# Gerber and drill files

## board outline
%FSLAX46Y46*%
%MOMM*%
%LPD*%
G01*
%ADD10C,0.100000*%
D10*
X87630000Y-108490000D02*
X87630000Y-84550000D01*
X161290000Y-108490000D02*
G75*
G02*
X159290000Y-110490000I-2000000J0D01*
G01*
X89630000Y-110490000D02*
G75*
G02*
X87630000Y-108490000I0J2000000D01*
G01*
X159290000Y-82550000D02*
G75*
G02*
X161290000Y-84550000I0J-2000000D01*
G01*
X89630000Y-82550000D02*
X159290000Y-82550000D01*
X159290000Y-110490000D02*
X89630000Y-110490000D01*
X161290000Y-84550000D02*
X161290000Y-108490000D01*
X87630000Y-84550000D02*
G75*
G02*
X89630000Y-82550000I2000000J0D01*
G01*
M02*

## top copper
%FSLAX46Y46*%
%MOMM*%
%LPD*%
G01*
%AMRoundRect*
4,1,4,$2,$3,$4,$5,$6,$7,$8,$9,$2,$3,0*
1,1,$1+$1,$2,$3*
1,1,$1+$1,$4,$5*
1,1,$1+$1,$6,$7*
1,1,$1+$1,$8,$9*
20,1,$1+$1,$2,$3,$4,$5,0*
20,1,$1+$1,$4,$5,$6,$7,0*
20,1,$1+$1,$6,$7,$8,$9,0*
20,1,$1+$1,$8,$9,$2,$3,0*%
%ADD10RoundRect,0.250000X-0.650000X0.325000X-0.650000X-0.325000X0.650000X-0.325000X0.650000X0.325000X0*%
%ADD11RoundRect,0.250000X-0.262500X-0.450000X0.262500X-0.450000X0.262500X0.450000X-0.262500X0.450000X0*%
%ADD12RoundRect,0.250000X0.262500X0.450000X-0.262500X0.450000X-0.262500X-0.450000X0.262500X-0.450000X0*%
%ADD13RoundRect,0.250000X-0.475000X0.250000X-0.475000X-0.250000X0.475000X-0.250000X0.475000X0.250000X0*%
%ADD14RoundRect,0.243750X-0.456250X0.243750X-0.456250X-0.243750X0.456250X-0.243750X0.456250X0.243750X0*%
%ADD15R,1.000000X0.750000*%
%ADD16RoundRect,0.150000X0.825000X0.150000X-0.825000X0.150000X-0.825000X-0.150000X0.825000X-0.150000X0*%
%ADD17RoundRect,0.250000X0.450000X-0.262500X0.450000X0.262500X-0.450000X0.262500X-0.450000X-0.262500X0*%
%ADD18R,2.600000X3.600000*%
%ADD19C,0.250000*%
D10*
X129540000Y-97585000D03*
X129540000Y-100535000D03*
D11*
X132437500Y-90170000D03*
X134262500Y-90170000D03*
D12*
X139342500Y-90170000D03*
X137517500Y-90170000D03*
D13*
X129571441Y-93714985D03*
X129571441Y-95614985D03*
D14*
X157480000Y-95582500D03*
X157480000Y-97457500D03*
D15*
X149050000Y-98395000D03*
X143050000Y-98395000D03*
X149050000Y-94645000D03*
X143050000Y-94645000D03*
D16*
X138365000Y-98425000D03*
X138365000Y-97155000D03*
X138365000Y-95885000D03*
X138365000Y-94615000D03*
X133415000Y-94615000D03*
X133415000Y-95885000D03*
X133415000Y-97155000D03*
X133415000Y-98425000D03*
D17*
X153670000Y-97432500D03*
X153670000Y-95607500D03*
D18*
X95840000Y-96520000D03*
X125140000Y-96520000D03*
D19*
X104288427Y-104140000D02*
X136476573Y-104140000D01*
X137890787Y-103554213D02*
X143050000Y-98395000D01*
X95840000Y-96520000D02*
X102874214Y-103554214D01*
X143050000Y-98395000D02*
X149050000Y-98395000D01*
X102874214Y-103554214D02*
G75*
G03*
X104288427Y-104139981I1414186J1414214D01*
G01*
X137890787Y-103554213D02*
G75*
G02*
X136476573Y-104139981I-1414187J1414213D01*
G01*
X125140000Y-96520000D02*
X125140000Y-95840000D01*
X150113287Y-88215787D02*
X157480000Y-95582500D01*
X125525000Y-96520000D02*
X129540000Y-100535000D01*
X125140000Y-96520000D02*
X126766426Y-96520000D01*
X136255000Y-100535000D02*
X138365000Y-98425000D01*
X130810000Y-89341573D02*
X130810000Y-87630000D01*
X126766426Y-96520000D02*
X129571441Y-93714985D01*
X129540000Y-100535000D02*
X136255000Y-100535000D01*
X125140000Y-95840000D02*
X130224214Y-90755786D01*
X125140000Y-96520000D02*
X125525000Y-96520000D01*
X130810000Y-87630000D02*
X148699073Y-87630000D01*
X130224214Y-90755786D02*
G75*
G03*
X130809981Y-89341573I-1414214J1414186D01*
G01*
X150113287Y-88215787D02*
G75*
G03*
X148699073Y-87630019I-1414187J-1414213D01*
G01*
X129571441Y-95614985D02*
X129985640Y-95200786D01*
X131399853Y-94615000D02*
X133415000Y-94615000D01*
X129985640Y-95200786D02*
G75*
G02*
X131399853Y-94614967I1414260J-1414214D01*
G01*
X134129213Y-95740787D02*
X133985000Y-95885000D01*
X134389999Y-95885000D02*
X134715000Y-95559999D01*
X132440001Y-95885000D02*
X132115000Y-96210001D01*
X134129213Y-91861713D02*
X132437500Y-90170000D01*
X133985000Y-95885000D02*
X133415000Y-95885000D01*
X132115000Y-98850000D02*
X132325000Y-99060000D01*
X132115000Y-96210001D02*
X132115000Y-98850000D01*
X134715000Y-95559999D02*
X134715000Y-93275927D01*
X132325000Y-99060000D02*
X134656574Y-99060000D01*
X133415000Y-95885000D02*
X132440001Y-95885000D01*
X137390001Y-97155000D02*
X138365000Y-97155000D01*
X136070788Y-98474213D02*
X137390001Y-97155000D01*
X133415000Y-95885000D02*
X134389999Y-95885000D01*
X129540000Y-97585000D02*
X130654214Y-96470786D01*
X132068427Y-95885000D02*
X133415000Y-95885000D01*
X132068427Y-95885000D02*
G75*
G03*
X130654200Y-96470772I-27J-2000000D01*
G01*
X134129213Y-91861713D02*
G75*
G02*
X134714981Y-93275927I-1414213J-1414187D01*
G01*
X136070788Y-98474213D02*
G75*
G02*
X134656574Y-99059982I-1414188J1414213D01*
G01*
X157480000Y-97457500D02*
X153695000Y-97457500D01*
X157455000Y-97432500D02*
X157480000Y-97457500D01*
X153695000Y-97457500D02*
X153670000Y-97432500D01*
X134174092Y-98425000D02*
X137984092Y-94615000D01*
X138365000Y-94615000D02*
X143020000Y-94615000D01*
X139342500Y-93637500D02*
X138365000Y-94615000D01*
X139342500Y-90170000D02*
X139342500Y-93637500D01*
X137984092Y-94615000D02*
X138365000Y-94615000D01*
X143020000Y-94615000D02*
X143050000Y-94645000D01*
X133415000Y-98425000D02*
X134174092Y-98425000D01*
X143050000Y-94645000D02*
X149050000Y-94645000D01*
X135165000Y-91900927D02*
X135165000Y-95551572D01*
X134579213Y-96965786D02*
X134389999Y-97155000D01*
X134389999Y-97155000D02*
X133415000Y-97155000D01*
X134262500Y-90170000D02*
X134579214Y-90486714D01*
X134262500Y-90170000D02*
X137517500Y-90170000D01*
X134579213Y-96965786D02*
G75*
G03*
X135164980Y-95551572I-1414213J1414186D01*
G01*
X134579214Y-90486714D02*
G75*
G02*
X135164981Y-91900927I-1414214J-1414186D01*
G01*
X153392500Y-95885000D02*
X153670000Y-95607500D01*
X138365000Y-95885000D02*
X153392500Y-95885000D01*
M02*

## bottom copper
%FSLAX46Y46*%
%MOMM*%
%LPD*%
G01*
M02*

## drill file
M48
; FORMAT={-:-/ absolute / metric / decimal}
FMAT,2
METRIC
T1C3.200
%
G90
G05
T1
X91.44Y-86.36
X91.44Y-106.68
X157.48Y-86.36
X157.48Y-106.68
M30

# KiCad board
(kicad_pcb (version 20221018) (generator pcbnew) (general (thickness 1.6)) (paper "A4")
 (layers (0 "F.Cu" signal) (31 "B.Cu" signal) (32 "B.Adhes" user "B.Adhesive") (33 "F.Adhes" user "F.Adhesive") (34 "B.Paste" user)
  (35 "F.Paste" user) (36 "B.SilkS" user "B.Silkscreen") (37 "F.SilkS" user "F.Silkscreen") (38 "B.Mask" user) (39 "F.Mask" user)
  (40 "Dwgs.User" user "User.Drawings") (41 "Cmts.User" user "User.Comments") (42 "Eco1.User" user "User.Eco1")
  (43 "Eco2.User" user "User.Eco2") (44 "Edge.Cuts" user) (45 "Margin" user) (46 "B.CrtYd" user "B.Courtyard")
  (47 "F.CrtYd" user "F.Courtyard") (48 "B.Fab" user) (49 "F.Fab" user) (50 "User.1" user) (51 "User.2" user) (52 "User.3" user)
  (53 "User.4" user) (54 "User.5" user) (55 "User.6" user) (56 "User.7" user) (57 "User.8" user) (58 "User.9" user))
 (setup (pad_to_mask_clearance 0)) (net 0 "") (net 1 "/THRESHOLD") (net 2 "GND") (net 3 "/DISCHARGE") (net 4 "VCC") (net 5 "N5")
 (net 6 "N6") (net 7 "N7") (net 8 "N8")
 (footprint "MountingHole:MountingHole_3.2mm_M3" (layer "F.Cu") (at 157.48 106.68)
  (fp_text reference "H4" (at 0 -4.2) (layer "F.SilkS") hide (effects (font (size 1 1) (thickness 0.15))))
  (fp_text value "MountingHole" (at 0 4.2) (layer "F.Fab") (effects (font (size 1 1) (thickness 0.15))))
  (pad "" np_thru_hole circle (at 0 0) (size 3.2 3.2) (drill 3.2) (layers "*.Cu" "*.Mask")))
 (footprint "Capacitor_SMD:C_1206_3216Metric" (layer "F.Cu") (at 129.54 99.06 -90)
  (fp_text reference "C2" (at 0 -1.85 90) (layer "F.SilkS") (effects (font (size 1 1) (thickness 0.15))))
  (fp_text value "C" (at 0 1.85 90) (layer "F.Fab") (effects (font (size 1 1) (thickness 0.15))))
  (pad "1" smd roundrect (at -1.475 0 270) (size 1.15 1.8) (layers "F.Cu" "F.Paste" "F.Mask") (roundrect_rratio 0.2173913043)
   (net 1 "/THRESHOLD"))
  (pad "2" smd roundrect (at 1.475 0 270) (size 1.15 1.8) (layers "F.Cu" "F.Paste" "F.Mask") (roundrect_rratio 0.2173913043) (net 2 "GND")))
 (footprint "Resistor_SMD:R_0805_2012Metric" (layer "F.Cu") (at 133.35 90.17)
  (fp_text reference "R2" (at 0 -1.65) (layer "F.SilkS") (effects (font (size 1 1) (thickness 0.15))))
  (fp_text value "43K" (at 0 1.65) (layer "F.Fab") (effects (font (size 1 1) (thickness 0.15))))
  (pad "1" smd roundrect (at -0.9125 0) (size 1.025 1.4) (layers "F.Cu" "F.Paste" "F.Mask") (roundrect_rratio 0.243902439)
   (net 1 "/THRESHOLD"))
  (pad "2" smd roundrect (at 0.9125 0) (size 1.025 1.4) (layers "F.Cu" "F.Paste" "F.Mask") (roundrect_rratio 0.243902439)
   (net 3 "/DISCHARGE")))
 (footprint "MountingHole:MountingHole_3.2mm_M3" (layer "F.Cu") (at 91.44 106.68)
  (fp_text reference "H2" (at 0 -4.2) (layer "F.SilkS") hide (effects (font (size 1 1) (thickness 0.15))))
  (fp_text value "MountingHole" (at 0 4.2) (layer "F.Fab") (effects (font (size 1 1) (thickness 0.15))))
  (pad "" np_thru_hole circle (at 0 0) (size 3.2 3.2) (drill 3.2) (layers "*.Cu" "*.Mask")))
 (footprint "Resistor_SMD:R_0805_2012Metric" (layer "F.Cu") (at 138.43 90.17 180)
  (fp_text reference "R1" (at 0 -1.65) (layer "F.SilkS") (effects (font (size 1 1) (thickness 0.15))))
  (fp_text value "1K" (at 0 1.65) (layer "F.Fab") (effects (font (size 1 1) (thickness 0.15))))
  (pad "1" smd roundrect (at -0.9125 0 180) (size 1.025 1.4) (layers "F.Cu" "F.Paste" "F.Mask") (roundrect_rratio 0.243902439) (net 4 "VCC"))
  (pad "2" smd roundrect (at 0.9125 0 180) (size 1.025 1.4) (layers "F.Cu" "F.Paste" "F.Mask") (roundrect_rratio 0.243902439)
   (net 3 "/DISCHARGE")))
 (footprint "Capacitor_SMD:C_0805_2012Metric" (layer "F.Cu") (at 129.571441 94.664985 -90)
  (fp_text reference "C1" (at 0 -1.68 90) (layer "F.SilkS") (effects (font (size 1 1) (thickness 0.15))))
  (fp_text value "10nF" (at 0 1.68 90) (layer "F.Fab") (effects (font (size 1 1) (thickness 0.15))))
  (pad "1" smd roundrect (at -0.95 0 270) (size 1 1.45) (layers "F.Cu" "F.Paste" "F.Mask") (roundrect_rratio 0.25) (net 2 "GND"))
  (pad "2" smd roundrect (at 0.95 0 270) (size 1 1.45) (layers "F.Cu" "F.Paste" "F.Mask") (roundrect_rratio 0.25) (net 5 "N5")))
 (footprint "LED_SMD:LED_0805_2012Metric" (layer "F.Cu") (at 157.48 96.52 -90)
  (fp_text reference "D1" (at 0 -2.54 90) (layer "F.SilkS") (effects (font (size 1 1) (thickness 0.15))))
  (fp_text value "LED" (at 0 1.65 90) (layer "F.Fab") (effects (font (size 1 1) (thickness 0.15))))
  (pad "1" smd roundrect (at -0.9375 0 270) (size 0.975 1.4) (layers "F.Cu" "F.Paste" "F.Mask") (roundrect_rratio 0.25) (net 2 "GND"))
  (pad "2" smd roundrect (at 0.9375 0 270) (size 0.975 1.4) (layers "F.Cu" "F.Paste" "F.Mask") (roundrect_rratio 0.25) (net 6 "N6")))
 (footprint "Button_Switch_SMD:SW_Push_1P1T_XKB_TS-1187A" (layer "F.Cu") (at 146.05 96.52 180)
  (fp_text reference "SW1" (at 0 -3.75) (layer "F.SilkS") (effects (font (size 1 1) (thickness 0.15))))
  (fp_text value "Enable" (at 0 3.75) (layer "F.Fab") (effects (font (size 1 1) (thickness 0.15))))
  (pad "1" smd rect (at -3 -1.875 180) (size 1 0.75) (layers "F.Cu" "F.Paste" "F.Mask") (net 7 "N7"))
  (pad "1" smd rect (at 3 -1.875 180) (size 1 0.75) (layers "F.Cu" "F.Paste" "F.Mask") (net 7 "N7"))
  (pad "2" smd rect (at -3 1.875 180) (size 1 0.75) (layers "F.Cu" "F.Paste" "F.Mask") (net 4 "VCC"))
  (pad "2" smd rect (at 3 1.875 180) (size 1 0.75) (layers "F.Cu" "F.Paste" "F.Mask") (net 4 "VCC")))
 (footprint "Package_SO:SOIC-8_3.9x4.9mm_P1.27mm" (layer "F.Cu") (at 135.89 96.52 180)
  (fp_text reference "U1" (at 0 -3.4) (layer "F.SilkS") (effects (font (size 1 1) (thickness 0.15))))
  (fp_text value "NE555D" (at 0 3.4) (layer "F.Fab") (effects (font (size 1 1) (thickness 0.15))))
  (pad "1" smd roundrect (at -2.475 -1.905 180) (size 1.95 0.6) (layers "F.Cu" "F.Paste" "F.Mask") (roundrect_rratio 0.25) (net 2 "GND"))
  (pad "2" smd roundrect (at -2.475 -0.635 180) (size 1.95 0.6) (layers "F.Cu" "F.Paste" "F.Mask") (roundrect_rratio 0.25)
   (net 1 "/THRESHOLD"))
  (pad "3" smd roundrect (at -2.475 0.635 180) (size 1.95 0.6) (layers "F.Cu" "F.Paste" "F.Mask") (roundrect_rratio 0.25) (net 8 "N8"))
  (pad "4" smd roundrect (at -2.475 1.905 180) (size 1.95 0.6) (layers "F.Cu" "F.Paste" "F.Mask") (roundrect_rratio 0.25) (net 4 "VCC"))
  (pad "5" smd roundrect (at 2.475 1.905 180) (size 1.95 0.6) (layers "F.Cu" "F.Paste" "F.Mask") (roundrect_rratio 0.25) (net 5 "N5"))
  (pad "6" smd roundrect (at 2.475 0.635 180) (size 1.95 0.6) (layers "F.Cu" "F.Paste" "F.Mask") (roundrect_rratio 0.25)
   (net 1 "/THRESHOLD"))
  (pad "7" smd roundrect (at 2.475 -0.635 180) (size 1.95 0.6) (layers "F.Cu" "F.Paste" "F.Mask") (roundrect_rratio 0.25)
   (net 3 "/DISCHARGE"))
  (pad "8" smd roundrect (at 2.475 -1.905 180) (size 1.95 0.6) (layers "F.Cu" "F.Paste" "F.Mask") (roundrect_rratio 0.25) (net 4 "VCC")))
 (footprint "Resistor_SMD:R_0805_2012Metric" (layer "F.Cu") (at 153.67 96.52 90)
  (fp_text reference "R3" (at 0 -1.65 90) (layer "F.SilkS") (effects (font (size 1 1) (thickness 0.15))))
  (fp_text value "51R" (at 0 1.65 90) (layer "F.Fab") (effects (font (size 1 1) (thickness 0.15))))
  (pad "1" smd roundrect (at -0.9125 0 90) (size 1.025 1.4) (layers "F.Cu" "F.Paste" "F.Mask") (roundrect_rratio 0.243902439) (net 6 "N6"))
  (pad "2" smd roundrect (at 0.9125 0 90) (size 1.025 1.4) (layers "F.Cu" "F.Paste" "F.Mask") (roundrect_rratio 0.243902439) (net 8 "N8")))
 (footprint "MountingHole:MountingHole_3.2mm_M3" (layer "F.Cu") (at 157.48 86.36)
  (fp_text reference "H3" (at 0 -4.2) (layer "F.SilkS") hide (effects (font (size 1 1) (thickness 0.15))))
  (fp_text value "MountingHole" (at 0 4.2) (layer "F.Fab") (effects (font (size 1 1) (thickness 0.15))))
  (pad "" np_thru_hole circle (at 0 0) (size 3.2 3.2) (drill 3.2) (layers "*.Cu" "*.Mask")))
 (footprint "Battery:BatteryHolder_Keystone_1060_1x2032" (layer "F.Cu") (at 110.49 96.52)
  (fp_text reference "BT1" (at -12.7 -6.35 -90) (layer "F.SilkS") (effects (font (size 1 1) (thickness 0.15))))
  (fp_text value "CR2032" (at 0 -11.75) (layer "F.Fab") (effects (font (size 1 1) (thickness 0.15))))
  (pad "1" smd rect (at -14.65 0 180) (size 2.6 3.6) (layers "F.Cu" "F.Paste" "F.Mask") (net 7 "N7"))
  (pad "2" smd rect (at 14.65 0 180) (size 2.6 3.6) (layers "F.Cu" "F.Paste" "F.Mask") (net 2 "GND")))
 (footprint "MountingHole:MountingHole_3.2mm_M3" (layer "F.Cu") (at 91.44 86.36)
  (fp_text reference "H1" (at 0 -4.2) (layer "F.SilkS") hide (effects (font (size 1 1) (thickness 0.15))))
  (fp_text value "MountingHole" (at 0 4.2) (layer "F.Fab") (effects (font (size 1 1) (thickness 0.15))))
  (pad "" np_thru_hole circle (at 0 0) (size 3.2 3.2) (drill 3.2) (layers "*.Cu" "*.Mask")))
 (gr_line (start 87.63 108.49) (end 87.63 84.55) (stroke (width 0.1) (type default)) (layer "Edge.Cuts"))
 (gr_arc (start 161.29 108.49) (mid 160.704214 109.904214) (end 159.29 110.49) (stroke (width 0.1) (type default)) (layer "Edge.Cuts"))
 (gr_arc (start 89.63 110.49) (mid 88.215786 109.904214) (end 87.63 108.49) (stroke (width 0.1) (type default)) (layer "Edge.Cuts"))
 (gr_arc (start 159.29 82.55) (mid 160.704214 83.135786) (end 161.29 84.55) (stroke (width 0.1) (type default)) (layer "Edge.Cuts"))
 (gr_line (start 89.63 82.55) (end 159.29 82.55) (stroke (width 0.1) (type default)) (layer "Edge.Cuts"))
 (gr_line (start 159.29 110.49) (end 89.63 110.49) (stroke (width 0.1) (type default)) (layer "Edge.Cuts"))
 (gr_line (start 161.29 84.55) (end 161.29 108.49) (stroke (width 0.1) (type default)) (layer "Edge.Cuts"))
 (gr_arc (start 87.63 84.55) (mid 88.215786 83.135786) (end 89.63 82.55) (stroke (width 0.1) (type default)) (layer "Edge.Cuts"))
 (segment (start 104.288427 104.14) (end 136.476573 104.14) (width 0.25) (layer "F.Cu") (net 7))
 (segment (start 137.890787 103.554213) (end 143.05 98.395) (width 0.25) (layer "F.Cu") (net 7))
 (segment (start 95.84 96.52) (end 102.874214 103.554214) (width 0.25) (layer "F.Cu") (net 7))
 (segment (start 143.05 98.395) (end 149.05 98.395) (width 0.25) (layer "F.Cu") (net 7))
 (arc (start 102.874214 103.554214) (mid 103.52306 103.987759) (end 104.288427 104.14) (width 0.25) (layer "F.Cu") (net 7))
 (arc (start 137.890787 103.554213) (mid 137.24194 103.987759) (end 136.476573 104.14) (width 0.25) (layer "F.Cu") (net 7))
 (segment (start 125.14 96.52) (end 125.14 95.84) (width 0.25) (layer "F.Cu") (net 2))
 (segment (start 150.113287 88.215787) (end 157.48 95.5825) (width 0.25) (layer "F.Cu") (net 2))
 (segment (start 125.525 96.52) (end 129.54 100.535) (width 0.25) (layer "F.Cu") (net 2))
 (segment (start 125.14 96.52) (end 126.766426 96.52) (width 0.25) (layer "F.Cu") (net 2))
 (segment (start 136.255 100.535) (end 138.365 98.425) (width 0.25) (layer "F.Cu") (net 2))
 (segment (start 130.81 89.341573) (end 130.81 87.63) (width 0.25) (layer "F.Cu") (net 2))
 (segment (start 126.766426 96.52) (end 129.571441 93.714985) (width 0.25) (layer "F.Cu") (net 2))
 (segment (start 129.54 100.535) (end 136.255 100.535) (width 0.25) (layer "F.Cu") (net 2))
 (segment (start 125.14 95.84) (end 130.224214 90.755786) (width 0.25) (layer "F.Cu") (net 2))
 (segment (start 125.14 96.52) (end 125.525 96.52) (width 0.25) (layer "F.Cu") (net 2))
 (segment (start 130.81 87.63) (end 148.699073 87.63) (width 0.25) (layer "F.Cu") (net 2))
 (arc (start 130.224214 90.755786) (mid 130.657759 90.10694) (end 130.81 89.341573) (width 0.25) (layer "F.Cu") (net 2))
 (arc (start 150.113287 88.215787) (mid 149.46444 87.782241) (end 148.699073 87.63) (width 0.25) (layer "F.Cu") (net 2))
 (segment (start 129.571441 95.614985) (end 129.98564 95.200786) (width 0.25) (layer "F.Cu") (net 5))
 (segment (start 131.399853 94.615) (end 133.415 94.615) (width 0.25) (layer "F.Cu") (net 5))
 (arc (start 129.98564 95.200786) (mid 130.634486 94.767241) (end 131.399853 94.615) (width 0.25) (layer "F.Cu") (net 5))
 (segment (start 134.129213 95.740787) (end 133.985 95.885) (width 0.25) (layer "F.Cu") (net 1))
 (segment (start 134.389999 95.885) (end 134.715 95.559999) (width 0.25) (layer "F.Cu") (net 1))
 (segment (start 132.440001 95.885) (end 132.115 96.210001) (width 0.25) (layer "F.Cu") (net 1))
 (segment (start 134.129213 91.861713) (end 132.4375 90.17) (width 0.25) (layer "F.Cu") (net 1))
 (segment (start 133.985 95.885) (end 133.415 95.885) (width 0.25) (layer "F.Cu") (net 1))
 (segment (start 132.115 98.85) (end 132.325 99.06) (width 0.25) (layer "F.Cu") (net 1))
 (segment (start 132.115 96.210001) (end 132.115 98.85) (width 0.25) (layer "F.Cu") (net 1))
 (segment (start 134.715 95.559999) (end 134.715 93.275927) (width 0.25) (layer "F.Cu") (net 1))
 (segment (start 132.325 99.06) (end 134.656574 99.06) (width 0.25) (layer "F.Cu") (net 1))
 (segment (start 133.415 95.885) (end 132.440001 95.885) (width 0.25) (layer "F.Cu") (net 1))
 (segment (start 137.390001 97.155) (end 138.365 97.155) (width 0.25) (layer "F.Cu") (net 1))
 (segment (start 136.070788 98.474213) (end 137.390001 97.155) (width 0.25) (layer "F.Cu") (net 1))
 (segment (start 133.415 95.885) (end 134.389999 95.885) (width 0.25) (layer "F.Cu") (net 1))
 (segment (start 129.54 97.585) (end 130.654214 96.470786) (width 0.25) (layer "F.Cu") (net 1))
 (segment (start 132.068427 95.885) (end 133.415 95.885) (width 0.25) (layer "F.Cu") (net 1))
 (arc (start 132.068427 95.885) (mid 131.30306 96.037241) (end 130.654214 96.470786) (width 0.25) (layer "F.Cu") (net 1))
 (arc (start 134.129213 91.861713) (mid 134.562759 92.51056) (end 134.715 93.275927) (width 0.25) (layer "F.Cu") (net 1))
 (arc (start 136.070788 98.474213) (mid 135.421941 98.907759) (end 134.656574 99.06) (width 0.25) (layer "F.Cu") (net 1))
 (segment (start 157.48 97.4575) (end 153.695 97.4575) (width 0.25) (layer "F.Cu") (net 6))
 (segment (start 157.455 97.4325) (end 157.48 97.4575) (width 0.25) (layer "F.Cu") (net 6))
 (segment (start 153.695 97.4575) (end 153.67 97.4325) (width 0.25) (layer "F.Cu") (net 6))
 (segment (start 134.174092 98.425) (end 137.984092 94.615) (width 0.25) (layer "F.Cu") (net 4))
 (segment (start 138.365 94.615) (end 143.02 94.615) (width 0.25) (layer "F.Cu") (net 4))
 (segment (start 139.3425 93.6375) (end 138.365 94.615) (width 0.25) (layer "F.Cu") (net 4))
 (segment (start 139.3425 90.17) (end 139.3425 93.6375) (width 0.25) (layer "F.Cu") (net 4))
 (segment (start 137.984092 94.615) (end 138.365 94.615) (width 0.25) (layer "F.Cu") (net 4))
 (segment (start 143.02 94.615) (end 143.05 94.645) (width 0.25) (layer "F.Cu") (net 4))
 (segment (start 133.415 98.425) (end 134.174092 98.425) (width 0.25) (layer "F.Cu") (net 4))
 (segment (start 143.05 94.645) (end 149.05 94.645) (width 0.25) (layer "F.Cu") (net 4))
 (segment (start 135.165 91.900927) (end 135.165 95.551572) (width 0.25) (layer "F.Cu") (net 3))
 (segment (start 134.579213 96.965786) (end 134.389999 97.155) (width 0.25) (layer "F.Cu") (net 3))
 (segment (start 134.389999 97.155) (end 133.415 97.155) (width 0.25) (layer "F.Cu") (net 3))
 (segment (start 134.2625 90.17) (end 134.579214 90.486714) (width 0.25) (layer "F.Cu") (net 3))
 (segment (start 134.2625 90.17) (end 137.5175 90.17) (width 0.25) (layer "F.Cu") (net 3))
 (arc (start 134.579213 96.965786) (mid 135.012759 96.316939) (end 135.165 95.551572) (width 0.25) (layer "F.Cu") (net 3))
 (arc (start 134.579214 90.486714) (mid 135.012759 91.13556) (end 135.165 91.900927) (width 0.25) (layer "F.Cu") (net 3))
 (segment (start 153.3925 95.885) (end 153.67 95.6075) (width 0.25) (layer "F.Cu") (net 8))
 (segment (start 138.365 95.885) (end 153.3925 95.885) (width 0.25) (layer "F.Cu") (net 8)))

